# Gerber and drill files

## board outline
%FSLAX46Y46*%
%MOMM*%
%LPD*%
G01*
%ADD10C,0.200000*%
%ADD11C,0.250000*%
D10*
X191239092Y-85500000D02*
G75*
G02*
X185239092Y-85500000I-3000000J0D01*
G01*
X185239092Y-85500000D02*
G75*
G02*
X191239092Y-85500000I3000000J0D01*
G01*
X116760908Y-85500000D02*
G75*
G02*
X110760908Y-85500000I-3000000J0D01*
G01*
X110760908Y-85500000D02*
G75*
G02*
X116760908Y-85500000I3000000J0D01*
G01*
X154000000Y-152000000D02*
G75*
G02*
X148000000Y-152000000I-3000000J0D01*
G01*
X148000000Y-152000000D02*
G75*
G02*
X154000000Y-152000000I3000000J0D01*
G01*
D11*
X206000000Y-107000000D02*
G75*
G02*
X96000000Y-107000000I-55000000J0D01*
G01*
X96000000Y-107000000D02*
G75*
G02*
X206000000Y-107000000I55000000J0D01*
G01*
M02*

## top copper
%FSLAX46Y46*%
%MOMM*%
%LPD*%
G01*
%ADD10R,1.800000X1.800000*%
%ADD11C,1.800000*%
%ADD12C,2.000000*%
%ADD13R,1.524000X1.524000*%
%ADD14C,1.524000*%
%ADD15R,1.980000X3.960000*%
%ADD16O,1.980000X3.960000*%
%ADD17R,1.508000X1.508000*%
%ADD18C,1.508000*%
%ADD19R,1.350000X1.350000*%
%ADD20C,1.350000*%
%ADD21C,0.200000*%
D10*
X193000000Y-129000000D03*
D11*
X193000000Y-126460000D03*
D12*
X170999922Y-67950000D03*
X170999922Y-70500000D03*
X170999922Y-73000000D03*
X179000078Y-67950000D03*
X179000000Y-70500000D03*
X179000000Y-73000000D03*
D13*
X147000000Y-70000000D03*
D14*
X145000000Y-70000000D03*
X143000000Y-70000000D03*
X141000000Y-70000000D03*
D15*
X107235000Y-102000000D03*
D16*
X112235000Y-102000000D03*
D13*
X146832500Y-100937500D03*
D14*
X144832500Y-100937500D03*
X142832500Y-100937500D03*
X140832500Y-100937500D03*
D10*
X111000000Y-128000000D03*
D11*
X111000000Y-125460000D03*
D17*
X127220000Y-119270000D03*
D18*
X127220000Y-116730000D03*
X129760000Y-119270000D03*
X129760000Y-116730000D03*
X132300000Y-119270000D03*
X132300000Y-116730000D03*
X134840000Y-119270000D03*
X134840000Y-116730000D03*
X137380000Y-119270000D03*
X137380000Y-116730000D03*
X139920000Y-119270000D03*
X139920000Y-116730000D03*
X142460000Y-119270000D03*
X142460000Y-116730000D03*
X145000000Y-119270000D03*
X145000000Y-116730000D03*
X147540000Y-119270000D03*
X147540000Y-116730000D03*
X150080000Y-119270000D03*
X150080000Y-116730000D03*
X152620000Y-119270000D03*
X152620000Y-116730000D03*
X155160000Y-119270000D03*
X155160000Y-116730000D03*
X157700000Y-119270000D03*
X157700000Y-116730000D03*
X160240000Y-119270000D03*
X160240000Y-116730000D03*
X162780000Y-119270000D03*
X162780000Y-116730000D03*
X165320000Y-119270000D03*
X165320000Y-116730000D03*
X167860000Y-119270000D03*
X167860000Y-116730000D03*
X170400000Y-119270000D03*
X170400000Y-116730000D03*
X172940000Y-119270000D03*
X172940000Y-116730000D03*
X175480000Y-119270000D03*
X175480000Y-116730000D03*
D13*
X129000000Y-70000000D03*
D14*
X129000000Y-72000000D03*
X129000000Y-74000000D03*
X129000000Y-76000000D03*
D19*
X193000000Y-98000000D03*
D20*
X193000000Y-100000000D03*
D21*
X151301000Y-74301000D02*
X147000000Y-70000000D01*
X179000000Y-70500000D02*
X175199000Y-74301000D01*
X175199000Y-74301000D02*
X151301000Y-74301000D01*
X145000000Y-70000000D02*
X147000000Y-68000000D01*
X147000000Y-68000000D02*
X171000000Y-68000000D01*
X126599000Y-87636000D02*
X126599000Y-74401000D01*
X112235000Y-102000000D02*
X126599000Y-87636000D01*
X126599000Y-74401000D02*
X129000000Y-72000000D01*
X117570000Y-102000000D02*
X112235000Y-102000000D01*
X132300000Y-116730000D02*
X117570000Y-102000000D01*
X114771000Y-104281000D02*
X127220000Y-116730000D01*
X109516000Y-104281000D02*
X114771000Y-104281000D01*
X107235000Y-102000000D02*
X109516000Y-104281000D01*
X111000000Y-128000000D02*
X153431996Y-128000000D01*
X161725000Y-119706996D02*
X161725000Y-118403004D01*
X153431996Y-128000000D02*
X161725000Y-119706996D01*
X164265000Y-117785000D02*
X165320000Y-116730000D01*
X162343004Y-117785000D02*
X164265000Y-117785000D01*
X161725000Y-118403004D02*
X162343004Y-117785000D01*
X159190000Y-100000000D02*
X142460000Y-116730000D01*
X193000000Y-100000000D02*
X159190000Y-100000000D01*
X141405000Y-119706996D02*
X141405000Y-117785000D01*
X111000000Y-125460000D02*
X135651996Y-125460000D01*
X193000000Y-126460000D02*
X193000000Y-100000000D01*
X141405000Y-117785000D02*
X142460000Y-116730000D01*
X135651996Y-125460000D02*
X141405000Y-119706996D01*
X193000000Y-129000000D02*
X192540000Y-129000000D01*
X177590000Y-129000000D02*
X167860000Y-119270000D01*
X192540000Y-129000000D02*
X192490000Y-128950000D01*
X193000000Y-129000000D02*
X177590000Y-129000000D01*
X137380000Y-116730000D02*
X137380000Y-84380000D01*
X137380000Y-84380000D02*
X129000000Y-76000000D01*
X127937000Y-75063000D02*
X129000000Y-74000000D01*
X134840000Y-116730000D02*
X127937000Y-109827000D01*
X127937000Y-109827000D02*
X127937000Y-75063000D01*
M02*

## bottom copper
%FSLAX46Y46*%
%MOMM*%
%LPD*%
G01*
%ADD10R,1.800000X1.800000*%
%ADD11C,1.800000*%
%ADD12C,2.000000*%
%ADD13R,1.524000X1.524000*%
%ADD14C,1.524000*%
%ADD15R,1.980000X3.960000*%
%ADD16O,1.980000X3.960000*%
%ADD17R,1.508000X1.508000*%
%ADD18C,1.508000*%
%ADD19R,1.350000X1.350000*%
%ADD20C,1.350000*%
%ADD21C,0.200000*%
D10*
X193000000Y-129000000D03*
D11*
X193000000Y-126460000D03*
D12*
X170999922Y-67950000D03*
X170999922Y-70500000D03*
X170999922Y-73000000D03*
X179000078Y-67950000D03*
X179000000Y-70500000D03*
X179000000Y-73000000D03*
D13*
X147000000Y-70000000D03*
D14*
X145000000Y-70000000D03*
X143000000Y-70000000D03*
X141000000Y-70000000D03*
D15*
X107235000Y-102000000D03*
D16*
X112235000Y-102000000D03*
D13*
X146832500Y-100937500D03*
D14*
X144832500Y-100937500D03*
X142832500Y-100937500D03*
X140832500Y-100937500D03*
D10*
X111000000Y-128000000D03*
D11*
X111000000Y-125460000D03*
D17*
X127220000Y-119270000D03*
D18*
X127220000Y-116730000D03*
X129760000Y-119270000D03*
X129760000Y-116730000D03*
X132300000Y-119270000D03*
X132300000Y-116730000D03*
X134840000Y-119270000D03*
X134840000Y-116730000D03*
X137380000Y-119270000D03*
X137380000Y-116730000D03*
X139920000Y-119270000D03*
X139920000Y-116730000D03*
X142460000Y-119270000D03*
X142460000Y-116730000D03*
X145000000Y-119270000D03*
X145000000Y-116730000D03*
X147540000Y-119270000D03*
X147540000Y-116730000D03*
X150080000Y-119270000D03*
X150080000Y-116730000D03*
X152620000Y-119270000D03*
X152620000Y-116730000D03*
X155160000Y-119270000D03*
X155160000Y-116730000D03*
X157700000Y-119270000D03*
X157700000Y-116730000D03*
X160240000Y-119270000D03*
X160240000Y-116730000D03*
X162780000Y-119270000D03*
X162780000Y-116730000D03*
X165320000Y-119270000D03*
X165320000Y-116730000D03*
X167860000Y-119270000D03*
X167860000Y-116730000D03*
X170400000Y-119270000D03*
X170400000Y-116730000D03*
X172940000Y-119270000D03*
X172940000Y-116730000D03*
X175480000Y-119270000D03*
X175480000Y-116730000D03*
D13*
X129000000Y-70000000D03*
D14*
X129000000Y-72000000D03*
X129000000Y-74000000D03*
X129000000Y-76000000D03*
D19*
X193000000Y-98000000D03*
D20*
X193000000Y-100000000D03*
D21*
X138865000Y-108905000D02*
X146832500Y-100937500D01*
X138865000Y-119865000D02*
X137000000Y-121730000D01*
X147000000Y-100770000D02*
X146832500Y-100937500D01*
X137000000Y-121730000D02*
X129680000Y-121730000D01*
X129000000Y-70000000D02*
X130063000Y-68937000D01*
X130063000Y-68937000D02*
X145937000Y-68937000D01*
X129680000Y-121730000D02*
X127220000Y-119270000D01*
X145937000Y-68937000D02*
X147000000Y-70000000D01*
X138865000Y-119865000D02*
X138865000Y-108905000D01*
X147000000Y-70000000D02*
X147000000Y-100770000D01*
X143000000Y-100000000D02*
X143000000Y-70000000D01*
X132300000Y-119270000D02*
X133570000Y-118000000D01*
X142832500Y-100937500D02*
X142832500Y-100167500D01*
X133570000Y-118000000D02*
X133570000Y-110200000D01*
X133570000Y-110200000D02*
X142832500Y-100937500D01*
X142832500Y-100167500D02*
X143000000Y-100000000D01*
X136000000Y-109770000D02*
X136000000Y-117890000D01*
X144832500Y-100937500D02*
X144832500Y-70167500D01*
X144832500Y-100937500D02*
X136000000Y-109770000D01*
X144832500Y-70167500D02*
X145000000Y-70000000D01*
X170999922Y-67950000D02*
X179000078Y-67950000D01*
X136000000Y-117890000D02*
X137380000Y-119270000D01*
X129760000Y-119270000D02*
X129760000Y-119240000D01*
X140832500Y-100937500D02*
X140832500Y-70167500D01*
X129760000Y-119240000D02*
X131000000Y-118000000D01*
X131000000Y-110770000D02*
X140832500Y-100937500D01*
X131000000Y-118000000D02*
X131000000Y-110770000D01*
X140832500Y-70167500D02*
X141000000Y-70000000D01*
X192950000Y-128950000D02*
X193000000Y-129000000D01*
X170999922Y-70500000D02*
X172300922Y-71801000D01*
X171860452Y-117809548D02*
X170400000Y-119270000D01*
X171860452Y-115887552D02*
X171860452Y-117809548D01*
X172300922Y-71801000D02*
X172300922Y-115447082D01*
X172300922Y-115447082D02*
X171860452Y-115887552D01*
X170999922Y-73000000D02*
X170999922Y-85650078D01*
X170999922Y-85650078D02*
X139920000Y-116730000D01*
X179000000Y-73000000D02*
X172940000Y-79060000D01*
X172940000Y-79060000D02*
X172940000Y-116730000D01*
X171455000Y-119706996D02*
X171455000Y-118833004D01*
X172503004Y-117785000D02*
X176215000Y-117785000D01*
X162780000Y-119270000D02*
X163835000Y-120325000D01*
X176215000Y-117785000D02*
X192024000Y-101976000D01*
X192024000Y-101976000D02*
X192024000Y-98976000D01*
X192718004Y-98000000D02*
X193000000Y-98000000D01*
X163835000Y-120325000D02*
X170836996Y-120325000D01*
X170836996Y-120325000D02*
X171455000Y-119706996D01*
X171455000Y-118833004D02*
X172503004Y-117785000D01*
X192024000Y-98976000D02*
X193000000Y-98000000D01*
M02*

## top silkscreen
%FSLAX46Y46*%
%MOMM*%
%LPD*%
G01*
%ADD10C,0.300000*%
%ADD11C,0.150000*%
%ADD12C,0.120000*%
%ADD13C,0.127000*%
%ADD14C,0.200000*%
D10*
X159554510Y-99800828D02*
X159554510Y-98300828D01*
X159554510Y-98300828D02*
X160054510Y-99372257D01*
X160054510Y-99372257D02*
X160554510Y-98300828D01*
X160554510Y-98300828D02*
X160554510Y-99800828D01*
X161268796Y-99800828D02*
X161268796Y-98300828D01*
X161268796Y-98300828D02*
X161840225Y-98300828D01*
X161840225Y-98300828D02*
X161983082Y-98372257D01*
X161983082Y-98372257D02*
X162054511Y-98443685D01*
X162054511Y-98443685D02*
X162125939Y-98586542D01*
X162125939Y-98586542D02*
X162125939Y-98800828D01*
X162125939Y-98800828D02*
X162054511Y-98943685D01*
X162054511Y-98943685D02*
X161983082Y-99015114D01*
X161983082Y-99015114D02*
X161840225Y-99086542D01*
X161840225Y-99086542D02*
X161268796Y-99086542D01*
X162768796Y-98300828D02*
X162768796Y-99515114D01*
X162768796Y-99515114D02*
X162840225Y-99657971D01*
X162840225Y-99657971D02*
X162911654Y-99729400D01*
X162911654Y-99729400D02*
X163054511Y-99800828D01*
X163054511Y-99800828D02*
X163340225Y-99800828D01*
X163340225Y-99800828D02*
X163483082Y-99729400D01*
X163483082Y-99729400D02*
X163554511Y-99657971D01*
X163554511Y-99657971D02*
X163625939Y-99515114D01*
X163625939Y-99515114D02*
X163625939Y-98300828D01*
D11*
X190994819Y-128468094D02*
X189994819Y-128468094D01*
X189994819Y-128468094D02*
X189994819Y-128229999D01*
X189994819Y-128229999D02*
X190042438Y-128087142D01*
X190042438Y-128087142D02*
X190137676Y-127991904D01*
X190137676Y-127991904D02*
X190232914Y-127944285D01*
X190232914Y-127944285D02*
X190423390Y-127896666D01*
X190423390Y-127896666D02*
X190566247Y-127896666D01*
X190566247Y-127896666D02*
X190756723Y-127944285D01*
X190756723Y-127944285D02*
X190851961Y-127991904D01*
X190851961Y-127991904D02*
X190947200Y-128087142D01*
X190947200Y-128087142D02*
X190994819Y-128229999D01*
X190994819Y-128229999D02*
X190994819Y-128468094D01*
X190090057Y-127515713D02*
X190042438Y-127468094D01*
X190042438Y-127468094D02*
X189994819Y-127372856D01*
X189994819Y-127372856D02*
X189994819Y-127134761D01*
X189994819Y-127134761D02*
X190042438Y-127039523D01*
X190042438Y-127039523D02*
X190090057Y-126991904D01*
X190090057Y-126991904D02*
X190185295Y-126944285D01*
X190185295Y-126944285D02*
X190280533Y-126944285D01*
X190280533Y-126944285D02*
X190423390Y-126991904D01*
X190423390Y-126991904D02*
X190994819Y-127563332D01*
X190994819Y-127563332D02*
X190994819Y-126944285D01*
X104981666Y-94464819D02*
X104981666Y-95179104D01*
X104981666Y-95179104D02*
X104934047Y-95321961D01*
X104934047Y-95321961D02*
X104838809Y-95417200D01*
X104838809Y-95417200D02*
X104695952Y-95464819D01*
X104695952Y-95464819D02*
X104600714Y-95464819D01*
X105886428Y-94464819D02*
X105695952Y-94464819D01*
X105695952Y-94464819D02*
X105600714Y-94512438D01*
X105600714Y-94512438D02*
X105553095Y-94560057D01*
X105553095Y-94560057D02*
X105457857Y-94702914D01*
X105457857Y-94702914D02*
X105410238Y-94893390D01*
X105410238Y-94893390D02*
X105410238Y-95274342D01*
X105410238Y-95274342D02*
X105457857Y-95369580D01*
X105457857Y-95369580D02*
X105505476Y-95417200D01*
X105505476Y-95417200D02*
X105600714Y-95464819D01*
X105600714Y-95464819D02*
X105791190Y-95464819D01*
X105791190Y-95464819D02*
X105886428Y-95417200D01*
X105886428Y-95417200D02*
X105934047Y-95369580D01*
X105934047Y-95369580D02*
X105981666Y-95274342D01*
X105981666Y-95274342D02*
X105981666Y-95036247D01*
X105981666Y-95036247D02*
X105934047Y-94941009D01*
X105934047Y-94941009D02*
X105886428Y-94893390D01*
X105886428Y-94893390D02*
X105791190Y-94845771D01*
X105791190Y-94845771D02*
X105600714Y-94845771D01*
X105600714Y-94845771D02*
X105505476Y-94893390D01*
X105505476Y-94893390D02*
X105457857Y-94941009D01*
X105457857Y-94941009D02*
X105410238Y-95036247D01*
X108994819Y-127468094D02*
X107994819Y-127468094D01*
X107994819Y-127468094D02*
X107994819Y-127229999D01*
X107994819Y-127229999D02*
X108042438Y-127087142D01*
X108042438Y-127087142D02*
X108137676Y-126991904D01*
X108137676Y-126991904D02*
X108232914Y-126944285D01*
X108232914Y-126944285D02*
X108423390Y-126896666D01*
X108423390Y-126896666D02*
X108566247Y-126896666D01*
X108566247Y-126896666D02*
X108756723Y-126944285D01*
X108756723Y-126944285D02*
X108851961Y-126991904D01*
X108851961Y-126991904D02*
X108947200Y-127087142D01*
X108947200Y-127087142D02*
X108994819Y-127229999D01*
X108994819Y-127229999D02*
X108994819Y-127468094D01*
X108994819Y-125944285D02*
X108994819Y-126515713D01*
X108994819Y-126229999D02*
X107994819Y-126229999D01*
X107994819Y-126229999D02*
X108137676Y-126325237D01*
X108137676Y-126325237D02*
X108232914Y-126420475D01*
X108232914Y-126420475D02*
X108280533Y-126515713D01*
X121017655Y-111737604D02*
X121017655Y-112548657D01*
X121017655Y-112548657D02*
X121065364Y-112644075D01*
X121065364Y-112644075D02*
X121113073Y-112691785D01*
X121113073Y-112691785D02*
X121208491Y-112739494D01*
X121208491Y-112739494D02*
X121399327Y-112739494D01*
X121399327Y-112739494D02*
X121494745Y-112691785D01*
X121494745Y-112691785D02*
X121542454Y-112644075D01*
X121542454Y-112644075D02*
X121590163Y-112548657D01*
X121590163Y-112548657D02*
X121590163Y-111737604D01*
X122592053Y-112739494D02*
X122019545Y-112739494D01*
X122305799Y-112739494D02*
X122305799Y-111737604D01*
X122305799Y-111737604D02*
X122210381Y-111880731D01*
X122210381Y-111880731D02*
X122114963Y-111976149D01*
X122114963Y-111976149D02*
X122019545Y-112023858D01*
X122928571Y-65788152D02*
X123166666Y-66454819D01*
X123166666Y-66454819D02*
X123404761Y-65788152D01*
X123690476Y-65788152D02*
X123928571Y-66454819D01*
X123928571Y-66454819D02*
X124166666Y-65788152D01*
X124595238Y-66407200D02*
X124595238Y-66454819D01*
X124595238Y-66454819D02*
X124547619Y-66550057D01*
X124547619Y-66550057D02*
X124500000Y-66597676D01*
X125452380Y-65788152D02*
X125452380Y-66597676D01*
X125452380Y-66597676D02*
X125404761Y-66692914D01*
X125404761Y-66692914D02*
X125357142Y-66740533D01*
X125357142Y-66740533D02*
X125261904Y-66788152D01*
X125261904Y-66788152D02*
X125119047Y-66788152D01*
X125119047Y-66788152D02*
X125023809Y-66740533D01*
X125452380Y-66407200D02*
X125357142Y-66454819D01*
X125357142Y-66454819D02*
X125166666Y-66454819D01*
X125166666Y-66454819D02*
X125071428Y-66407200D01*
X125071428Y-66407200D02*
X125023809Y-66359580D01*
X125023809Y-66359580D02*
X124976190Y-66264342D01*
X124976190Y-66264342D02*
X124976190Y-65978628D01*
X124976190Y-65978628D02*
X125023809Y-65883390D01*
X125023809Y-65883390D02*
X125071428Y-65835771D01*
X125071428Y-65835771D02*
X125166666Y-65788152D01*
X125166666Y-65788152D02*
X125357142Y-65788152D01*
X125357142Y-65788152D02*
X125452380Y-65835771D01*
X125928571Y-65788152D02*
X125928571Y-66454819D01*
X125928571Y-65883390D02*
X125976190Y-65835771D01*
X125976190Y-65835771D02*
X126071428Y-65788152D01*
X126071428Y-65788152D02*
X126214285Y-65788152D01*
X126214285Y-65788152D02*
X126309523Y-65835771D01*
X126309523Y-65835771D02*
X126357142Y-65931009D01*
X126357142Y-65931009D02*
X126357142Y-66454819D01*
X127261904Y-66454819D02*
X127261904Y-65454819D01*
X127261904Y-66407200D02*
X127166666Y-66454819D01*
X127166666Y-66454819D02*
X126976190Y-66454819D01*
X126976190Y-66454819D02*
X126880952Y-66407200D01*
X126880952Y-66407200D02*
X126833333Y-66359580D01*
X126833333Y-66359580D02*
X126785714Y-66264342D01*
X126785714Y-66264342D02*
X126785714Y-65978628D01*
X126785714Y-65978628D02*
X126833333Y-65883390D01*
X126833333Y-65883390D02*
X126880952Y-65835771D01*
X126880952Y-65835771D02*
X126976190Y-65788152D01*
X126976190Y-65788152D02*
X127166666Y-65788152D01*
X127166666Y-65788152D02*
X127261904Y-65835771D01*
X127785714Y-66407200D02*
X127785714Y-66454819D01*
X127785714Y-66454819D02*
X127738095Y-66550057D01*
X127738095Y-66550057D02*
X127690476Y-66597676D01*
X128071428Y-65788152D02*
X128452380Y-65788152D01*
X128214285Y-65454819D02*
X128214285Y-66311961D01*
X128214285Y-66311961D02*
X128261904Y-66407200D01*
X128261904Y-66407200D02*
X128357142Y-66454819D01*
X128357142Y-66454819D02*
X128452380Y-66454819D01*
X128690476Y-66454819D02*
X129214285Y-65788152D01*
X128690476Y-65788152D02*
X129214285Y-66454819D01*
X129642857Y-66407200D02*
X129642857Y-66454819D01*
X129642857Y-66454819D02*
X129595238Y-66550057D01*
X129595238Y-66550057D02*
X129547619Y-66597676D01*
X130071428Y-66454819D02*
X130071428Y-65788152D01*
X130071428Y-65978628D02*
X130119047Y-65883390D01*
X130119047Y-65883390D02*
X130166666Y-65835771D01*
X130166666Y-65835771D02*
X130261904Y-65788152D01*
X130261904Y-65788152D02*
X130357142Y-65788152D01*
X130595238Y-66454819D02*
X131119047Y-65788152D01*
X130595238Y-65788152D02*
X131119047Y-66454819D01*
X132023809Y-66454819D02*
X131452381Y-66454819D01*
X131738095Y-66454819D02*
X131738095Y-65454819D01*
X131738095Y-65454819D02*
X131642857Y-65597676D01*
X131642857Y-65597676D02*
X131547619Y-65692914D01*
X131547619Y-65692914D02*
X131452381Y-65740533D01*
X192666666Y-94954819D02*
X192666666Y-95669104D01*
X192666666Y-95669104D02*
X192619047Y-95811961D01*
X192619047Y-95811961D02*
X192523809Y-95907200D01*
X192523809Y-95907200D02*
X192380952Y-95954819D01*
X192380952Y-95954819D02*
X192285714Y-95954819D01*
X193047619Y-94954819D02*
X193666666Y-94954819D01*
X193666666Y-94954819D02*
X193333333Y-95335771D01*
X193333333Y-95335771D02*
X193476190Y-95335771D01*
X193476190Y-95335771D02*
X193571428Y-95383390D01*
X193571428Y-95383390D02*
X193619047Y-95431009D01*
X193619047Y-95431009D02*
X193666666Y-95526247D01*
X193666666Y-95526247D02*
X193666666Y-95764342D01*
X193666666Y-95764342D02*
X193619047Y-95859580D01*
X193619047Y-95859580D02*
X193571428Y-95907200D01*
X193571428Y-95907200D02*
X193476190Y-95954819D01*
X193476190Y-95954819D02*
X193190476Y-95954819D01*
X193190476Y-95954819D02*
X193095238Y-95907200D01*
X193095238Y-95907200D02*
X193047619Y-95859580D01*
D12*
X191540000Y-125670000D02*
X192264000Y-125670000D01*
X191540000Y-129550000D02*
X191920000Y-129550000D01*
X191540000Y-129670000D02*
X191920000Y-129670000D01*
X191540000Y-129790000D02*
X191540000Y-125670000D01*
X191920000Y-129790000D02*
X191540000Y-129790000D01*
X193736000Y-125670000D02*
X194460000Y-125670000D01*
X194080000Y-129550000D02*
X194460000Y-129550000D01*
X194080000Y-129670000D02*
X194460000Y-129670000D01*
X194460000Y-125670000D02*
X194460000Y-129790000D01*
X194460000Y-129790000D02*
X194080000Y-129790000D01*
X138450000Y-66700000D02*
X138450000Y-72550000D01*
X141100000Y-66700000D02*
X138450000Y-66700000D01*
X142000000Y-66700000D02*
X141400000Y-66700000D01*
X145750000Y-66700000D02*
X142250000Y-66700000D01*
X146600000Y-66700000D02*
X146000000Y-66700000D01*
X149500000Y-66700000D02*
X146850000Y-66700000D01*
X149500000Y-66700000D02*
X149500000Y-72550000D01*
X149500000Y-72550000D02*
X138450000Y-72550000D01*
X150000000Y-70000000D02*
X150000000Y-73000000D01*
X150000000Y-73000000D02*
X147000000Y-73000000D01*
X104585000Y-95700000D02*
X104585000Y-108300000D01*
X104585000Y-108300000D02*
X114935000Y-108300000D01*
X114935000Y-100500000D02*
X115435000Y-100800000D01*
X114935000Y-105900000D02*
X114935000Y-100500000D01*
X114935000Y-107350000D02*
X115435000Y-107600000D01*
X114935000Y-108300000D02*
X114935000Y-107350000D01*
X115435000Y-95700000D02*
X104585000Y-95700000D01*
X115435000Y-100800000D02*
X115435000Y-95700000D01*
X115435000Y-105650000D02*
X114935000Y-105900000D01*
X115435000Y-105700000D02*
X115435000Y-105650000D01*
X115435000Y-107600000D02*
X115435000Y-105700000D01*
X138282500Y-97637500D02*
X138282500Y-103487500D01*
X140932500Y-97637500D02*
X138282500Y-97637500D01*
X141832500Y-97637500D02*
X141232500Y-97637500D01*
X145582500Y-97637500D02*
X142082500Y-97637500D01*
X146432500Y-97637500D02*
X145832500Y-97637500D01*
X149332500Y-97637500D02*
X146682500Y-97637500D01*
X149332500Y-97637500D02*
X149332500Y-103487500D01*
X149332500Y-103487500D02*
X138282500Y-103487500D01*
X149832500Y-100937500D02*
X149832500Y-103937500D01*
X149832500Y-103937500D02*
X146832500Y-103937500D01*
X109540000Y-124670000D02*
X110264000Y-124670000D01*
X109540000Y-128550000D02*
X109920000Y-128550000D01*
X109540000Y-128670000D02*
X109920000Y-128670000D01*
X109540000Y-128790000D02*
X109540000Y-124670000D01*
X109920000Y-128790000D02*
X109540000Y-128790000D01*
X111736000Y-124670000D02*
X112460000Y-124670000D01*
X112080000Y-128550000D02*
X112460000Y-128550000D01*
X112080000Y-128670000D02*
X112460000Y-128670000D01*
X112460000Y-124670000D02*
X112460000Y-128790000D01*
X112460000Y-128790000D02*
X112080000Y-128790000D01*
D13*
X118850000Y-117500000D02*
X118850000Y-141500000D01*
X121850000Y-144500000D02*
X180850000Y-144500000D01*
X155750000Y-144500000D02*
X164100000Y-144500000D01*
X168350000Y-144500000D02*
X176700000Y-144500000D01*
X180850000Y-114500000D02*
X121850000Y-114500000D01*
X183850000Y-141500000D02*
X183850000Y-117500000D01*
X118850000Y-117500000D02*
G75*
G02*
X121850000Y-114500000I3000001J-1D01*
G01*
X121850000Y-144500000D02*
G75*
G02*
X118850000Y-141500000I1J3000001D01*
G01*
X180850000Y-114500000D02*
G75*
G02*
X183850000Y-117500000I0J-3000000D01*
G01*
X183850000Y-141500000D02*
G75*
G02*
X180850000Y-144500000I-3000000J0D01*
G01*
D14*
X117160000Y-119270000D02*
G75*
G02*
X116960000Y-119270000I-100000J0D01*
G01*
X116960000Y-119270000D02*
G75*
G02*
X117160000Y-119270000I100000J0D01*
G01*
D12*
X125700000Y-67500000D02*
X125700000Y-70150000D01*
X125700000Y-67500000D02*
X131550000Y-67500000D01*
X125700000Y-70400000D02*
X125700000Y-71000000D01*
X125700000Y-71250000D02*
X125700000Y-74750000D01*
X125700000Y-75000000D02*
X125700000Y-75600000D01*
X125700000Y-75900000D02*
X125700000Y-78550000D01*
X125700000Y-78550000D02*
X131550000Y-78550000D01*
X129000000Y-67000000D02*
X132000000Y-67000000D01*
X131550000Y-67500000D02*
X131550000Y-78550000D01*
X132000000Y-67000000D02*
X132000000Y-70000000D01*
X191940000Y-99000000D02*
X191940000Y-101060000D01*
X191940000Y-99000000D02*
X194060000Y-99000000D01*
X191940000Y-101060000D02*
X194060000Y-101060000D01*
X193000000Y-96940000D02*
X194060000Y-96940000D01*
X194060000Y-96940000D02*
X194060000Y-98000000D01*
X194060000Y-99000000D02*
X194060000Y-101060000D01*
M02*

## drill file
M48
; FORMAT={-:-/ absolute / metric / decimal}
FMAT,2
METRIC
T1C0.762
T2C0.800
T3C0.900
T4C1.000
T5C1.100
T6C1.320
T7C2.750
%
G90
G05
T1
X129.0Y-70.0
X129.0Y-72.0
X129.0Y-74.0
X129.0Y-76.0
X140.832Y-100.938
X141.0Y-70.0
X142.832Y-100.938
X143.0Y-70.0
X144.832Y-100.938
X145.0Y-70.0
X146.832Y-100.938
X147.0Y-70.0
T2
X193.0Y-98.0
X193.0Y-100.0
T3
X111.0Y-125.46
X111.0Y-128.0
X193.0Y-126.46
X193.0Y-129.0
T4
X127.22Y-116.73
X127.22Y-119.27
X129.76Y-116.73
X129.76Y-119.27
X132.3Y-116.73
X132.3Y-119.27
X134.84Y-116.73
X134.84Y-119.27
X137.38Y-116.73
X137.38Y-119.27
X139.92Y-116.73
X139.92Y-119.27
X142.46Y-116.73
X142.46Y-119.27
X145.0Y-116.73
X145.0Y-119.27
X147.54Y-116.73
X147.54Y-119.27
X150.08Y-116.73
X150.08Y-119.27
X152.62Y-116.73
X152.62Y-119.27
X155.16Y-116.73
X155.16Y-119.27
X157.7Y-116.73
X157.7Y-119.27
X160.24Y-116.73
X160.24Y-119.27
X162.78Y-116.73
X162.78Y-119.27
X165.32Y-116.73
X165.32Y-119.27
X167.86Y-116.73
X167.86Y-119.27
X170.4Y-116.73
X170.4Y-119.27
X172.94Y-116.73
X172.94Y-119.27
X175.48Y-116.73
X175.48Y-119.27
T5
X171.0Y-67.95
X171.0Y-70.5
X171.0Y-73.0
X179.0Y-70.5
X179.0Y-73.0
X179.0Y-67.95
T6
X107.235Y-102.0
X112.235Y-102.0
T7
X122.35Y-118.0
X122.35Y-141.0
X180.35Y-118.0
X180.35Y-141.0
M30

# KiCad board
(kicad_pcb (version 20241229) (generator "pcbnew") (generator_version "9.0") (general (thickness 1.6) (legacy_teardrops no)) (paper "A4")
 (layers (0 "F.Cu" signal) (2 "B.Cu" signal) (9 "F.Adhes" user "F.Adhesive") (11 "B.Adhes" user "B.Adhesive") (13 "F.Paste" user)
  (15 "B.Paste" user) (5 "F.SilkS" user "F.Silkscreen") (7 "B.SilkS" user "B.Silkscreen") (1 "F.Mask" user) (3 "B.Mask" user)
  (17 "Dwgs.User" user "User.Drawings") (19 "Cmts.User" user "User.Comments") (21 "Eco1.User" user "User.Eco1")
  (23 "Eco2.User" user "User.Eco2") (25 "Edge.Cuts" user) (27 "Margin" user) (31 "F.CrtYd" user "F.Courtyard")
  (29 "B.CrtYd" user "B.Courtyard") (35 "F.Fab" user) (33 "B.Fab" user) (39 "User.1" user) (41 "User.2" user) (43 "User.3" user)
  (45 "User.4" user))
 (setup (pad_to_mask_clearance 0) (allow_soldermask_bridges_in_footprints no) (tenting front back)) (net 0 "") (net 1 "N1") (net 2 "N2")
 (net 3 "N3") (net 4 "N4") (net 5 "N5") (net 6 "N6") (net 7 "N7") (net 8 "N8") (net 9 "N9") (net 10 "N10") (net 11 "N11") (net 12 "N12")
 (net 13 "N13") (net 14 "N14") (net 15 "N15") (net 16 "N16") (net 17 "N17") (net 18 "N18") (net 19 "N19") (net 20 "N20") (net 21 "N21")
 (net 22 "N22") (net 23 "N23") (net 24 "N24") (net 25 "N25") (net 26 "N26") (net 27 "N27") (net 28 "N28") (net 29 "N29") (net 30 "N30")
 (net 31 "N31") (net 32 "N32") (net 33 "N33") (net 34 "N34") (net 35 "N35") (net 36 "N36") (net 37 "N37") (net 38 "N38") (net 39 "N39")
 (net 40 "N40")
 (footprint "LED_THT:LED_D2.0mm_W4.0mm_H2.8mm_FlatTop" (layer "F.Cu") (at 193 129 90)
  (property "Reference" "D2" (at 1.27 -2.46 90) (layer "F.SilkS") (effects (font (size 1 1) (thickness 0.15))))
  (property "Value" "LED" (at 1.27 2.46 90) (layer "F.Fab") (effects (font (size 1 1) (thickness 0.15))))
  (fp_line (start 3.33 -1.46) (end 3.33 -0.736) (stroke (width 0.12) (type solid)) (layer "F.SilkS"))
  (fp_line (start -0.55 -1.46) (end -0.55 -1.08) (stroke (width 0.12) (type solid)) (layer "F.SilkS"))
  (fp_line (start -0.67 -1.46) (end -0.67 -1.08) (stroke (width 0.12) (type solid)) (layer "F.SilkS"))
  (fp_line (start -0.79 -1.46) (end 3.33 -1.46) (stroke (width 0.12) (type solid)) (layer "F.SilkS"))
  (fp_line (start -0.79 -1.08) (end -0.79 -1.46) (stroke (width 0.12) (type solid)) (layer "F.SilkS"))
  (fp_line (start 3.33 0.736) (end 3.33 1.46) (stroke (width 0.12) (type solid)) (layer "F.SilkS"))
  (fp_line (start -0.55 1.08) (end -0.55 1.46) (stroke (width 0.12) (type solid)) (layer "F.SilkS"))
  (fp_line (start -0.67 1.08) (end -0.67 1.46) (stroke (width 0.12) (type solid)) (layer "F.SilkS"))
  (fp_line (start 3.33 1.46) (end -0.79 1.46) (stroke (width 0.12) (type solid)) (layer "F.SilkS"))
  (fp_line (start -0.79 1.46) (end -0.79 1.08) (stroke (width 0.12) (type solid)) (layer "F.SilkS"))
  (pad "1" thru_hole rect (at 0 0 90) (size 1.8 1.8) (drill 0.9) (layers "*.Cu" "*.Mask") (remove_unused_layers no) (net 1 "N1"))
  (pad "2" thru_hole circle (at 2.54 0 90) (size 1.8 1.8) (drill 0.9) (layers "*.Cu" "*.Mask") (remove_unused_layers no) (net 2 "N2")))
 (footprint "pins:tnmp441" (layer "F.Cu") (at 174.999922 70.5)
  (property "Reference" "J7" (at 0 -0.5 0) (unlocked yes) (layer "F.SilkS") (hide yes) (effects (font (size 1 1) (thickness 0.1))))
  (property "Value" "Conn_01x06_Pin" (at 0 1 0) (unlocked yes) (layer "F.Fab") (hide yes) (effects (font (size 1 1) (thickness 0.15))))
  (pad "1" thru_hole circle (at -4 -2.55) (size 2 2) (drill 1.1) (layers "*.Cu" "*.Mask") (remove_unused_layers no) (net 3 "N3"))
  (pad "2" thru_hole circle (at -4 0) (size 2 2) (drill 1.1) (layers "*.Cu" "*.Mask") (remove_unused_layers no) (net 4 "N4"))
  (pad "3" thru_hole circle (at -4 2.5) (size 2 2) (drill 1.1) (layers "*.Cu" "*.Mask") (remove_unused_layers no) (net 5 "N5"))
  (pad "4" thru_hole circle (at 4.000156 -2.55) (size 2 2) (drill 1.1) (layers "*.Cu" "*.Mask") (remove_unused_layers no) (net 3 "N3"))
  (pad "5" thru_hole circle (at 4.000078 0) (size 2 2) (drill 1.1) (layers "*.Cu" "*.Mask") (remove_unused_layers no) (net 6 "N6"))
  (pad "6" thru_hole circle (at 4.000078 2.5) (size 2 2) (drill 1.1) (layers "*.Cu" "*.Mask") (remove_unused_layers no) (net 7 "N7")))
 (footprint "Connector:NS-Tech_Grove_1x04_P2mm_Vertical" (layer "F.Cu") (at 147 70 -90)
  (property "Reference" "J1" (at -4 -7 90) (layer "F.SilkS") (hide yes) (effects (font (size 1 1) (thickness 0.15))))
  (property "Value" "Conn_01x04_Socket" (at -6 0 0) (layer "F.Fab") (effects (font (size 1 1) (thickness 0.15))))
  (fp_line (start -3.3 8.55) (end 2.55 8.55) (stroke (width 0.12) (type solid)) (layer "F.SilkS"))
  (fp_line (start -3.3 5.9) (end -3.3 8.55) (stroke (width 0.12) (type solid)) (layer "F.SilkS"))
  (fp_line (start -3.3 5) (end -3.3 5.6) (stroke (width 0.12) (type solid)) (layer "F.SilkS"))
  (fp_line (start -3.3 1.25) (end -3.3 4.75) (stroke (width 0.12) (type solid)) (layer "F.SilkS"))
  (fp_line (start -3.3 0.4) (end -3.3 1) (stroke (width 0.12) (type solid)) (layer "F.SilkS"))
  (fp_line (start -3.3 -2.5) (end -3.3 0.15) (stroke (width 0.12) (type solid)) (layer "F.SilkS"))
  (fp_line (start -3.3 -2.5) (end 2.55 -2.5) (stroke (width 0.12) (type solid)) (layer "F.SilkS"))
  (fp_line (start 2.55 -2.5) (end 2.55 8.55) (stroke (width 0.12) (type solid)) (layer "F.SilkS"))
  (fp_line (start 0 -3) (end 3 -3) (stroke (width 0.12) (type solid)) (layer "F.SilkS"))
  (fp_line (start 3 -3) (end 3 0) (stroke (width 0.12) (type solid)) (layer "F.SilkS"))
  (pad "1" thru_hole rect (at 0 0 270) (size 1.524 1.524) (drill 0.762) (layers "*.Cu" "*.Mask") (remove_unused_layers no) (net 6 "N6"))
  (pad "2" thru_hole circle (at 0 2 270) (size 1.524 1.524) (drill 0.762) (layers "*.Cu" "*.Mask") (remove_unused_layers no) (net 3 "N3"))
  (pad "3" thru_hole circle (at 0 4 270) (size 1.524 1.524) (drill 0.762) (layers "*.Cu" "*.Mask") (remove_unused_layers no) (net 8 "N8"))
  (pad "4" thru_hole circle (at 0 6 270) (size 1.524 1.524) (drill 0.762) (layers "*.Cu" "*.Mask") (remove_unused_layers no) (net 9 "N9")))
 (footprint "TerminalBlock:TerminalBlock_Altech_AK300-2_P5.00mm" (layer "F.Cu") (at 107.235 102)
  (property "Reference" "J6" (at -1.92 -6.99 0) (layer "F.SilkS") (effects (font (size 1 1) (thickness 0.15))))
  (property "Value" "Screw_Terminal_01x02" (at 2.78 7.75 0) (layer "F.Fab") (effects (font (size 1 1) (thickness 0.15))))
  (fp_line (start -2.65 -6.3) (end -2.65 6.3) (stroke (width 0.12) (type solid)) (layer "F.SilkS"))
  (fp_line (start -2.65 6.3) (end 7.7 6.3) (stroke (width 0.12) (type solid)) (layer "F.SilkS"))
  (fp_line (start 7.7 -1.5) (end 8.2 -1.2) (stroke (width 0.12) (type solid)) (layer "F.SilkS"))
  (fp_line (start 7.7 3.9) (end 7.7 -1.5) (stroke (width 0.12) (type solid)) (layer "F.SilkS"))
  (fp_line (start 7.7 5.35) (end 8.2 5.6) (stroke (width 0.12) (type solid)) (layer "F.SilkS"))
  (fp_line (start 7.7 6.3) (end 7.7 5.35) (stroke (width 0.12) (type solid)) (layer "F.SilkS"))
  (fp_line (start 8.2 -6.3) (end -2.65 -6.3) (stroke (width 0.12) (type solid)) (layer "F.SilkS"))
  (fp_line (start 8.2 -1.2) (end 8.2 -6.3) (stroke (width 0.12) (type solid)) (layer "F.SilkS"))
  (fp_line (start 8.2 3.65) (end 7.7 3.9) (stroke (width 0.12) (type solid)) (layer "F.SilkS"))
  (fp_line (start 8.2 3.7) (end 8.2 3.65) (stroke (width 0.12) (type solid)) (layer "F.SilkS"))
  (fp_line (start 8.2 5.6) (end 8.2 3.7) (stroke (width 0.12) (type solid)) (layer "F.SilkS"))
  (pad "1" thru_hole rect (at 0 0) (size 1.98 3.96) (drill 1.32) (layers "*.Cu" "*.Mask") (remove_unused_layers no) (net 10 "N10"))
  (pad "2" thru_hole oval (at 5 0) (size 1.98 3.96) (drill 1.32) (layers "*.Cu" "*.Mask") (remove_unused_layers no) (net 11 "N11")))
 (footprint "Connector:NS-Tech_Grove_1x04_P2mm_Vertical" (layer "F.Cu") (at 146.8325 100.9375 -90)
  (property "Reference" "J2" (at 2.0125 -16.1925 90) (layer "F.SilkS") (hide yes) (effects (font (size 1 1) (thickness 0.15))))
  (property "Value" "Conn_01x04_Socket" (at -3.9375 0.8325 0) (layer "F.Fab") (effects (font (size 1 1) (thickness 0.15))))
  (fp_line (start -3.3 8.55) (end 2.55 8.55) (stroke (width 0.12) (type solid)) (layer "F.SilkS"))
  (fp_line (start -3.3 5.9) (end -3.3 8.55) (stroke (width 0.12) (type solid)) (layer "F.SilkS"))
  (fp_line (start -3.3 5) (end -3.3 5.6) (stroke (width 0.12) (type solid)) (layer "F.SilkS"))
  (fp_line (start -3.3 1.25) (end -3.3 4.75) (stroke (width 0.12) (type solid)) (layer "F.SilkS"))
  (fp_line (start -3.3 0.4) (end -3.3 1) (stroke (width 0.12) (type solid)) (layer "F.SilkS"))
  (fp_line (start -3.3 -2.5) (end -3.3 0.15) (stroke (width 0.12) (type solid)) (layer "F.SilkS"))
  (fp_line (start -3.3 -2.5) (end 2.55 -2.5) (stroke (width 0.12) (type solid)) (layer "F.SilkS"))
  (fp_line (start 2.55 -2.5) (end 2.55 8.55) (stroke (width 0.12) (type solid)) (layer "F.SilkS"))
  (fp_line (start 0 -3) (end 3 -3) (stroke (width 0.12) (type solid)) (layer "F.SilkS"))
  (fp_line (start 3 -3) (end 3 0) (stroke (width 0.12) (type solid)) (layer "F.SilkS"))
  (pad "1" thru_hole rect (at 0 0 270) (size 1.524 1.524) (drill 0.762) (layers "*.Cu" "*.Mask") (remove_unused_layers no) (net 6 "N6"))
  (pad "2" thru_hole circle (at 0 2 270) (size 1.524 1.524) (drill 0.762) (layers "*.Cu" "*.Mask") (remove_unused_layers no) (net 3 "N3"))
  (pad "3" thru_hole circle (at 0 4 270) (size 1.524 1.524) (drill 0.762) (layers "*.Cu" "*.Mask") (remove_unused_layers no) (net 8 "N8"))
  (pad "4" thru_hole circle (at 0 6 270) (size 1.524 1.524) (drill 0.762) (layers "*.Cu" "*.Mask") (remove_unused_layers no) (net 9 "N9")))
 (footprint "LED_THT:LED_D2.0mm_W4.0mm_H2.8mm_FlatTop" (layer "F.Cu") (at 111 128 90)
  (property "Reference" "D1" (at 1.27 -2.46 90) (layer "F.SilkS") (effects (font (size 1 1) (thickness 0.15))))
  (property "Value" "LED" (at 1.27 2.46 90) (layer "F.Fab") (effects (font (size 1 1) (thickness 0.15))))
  (fp_line (start 3.33 -1.46) (end 3.33 -0.736) (stroke (width 0.12) (type solid)) (layer "F.SilkS"))
  (fp_line (start -0.55 -1.46) (end -0.55 -1.08) (stroke (width 0.12) (type solid)) (layer "F.SilkS"))
  (fp_line (start -0.67 -1.46) (end -0.67 -1.08) (stroke (width 0.12) (type solid)) (layer "F.SilkS"))
  (fp_line (start -0.79 -1.46) (end 3.33 -1.46) (stroke (width 0.12) (type solid)) (layer "F.SilkS"))
  (fp_line (start -0.79 -1.08) (end -0.79 -1.46) (stroke (width 0.12) (type solid)) (layer "F.SilkS"))
  (fp_line (start 3.33 0.736) (end 3.33 1.46) (stroke (width 0.12) (type solid)) (layer "F.SilkS"))
  (fp_line (start -0.55 1.08) (end -0.55 1.46) (stroke (width 0.12) (type solid)) (layer "F.SilkS"))
  (fp_line (start -0.67 1.08) (end -0.67 1.46) (stroke (width 0.12) (type solid)) (layer "F.SilkS"))
  (fp_line (start 3.33 1.46) (end -0.79 1.46) (stroke (width 0.12) (type solid)) (layer "F.SilkS"))
  (fp_line (start -0.79 1.46) (end -0.79 1.08) (stroke (width 0.12) (type solid)) (layer "F.SilkS"))
  (pad "1" thru_hole rect (at 0 0 90) (size 1.8 1.8) (drill 0.9) (layers "*.Cu" "*.Mask") (remove_unused_layers no) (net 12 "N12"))
  (pad "2" thru_hole circle (at 2.54 0 90) (size 1.8 1.8) (drill 0.9) (layers "*.Cu" "*.Mask") (remove_unused_layers no) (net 2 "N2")))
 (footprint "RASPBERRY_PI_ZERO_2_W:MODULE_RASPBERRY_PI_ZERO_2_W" (layer "F.Cu") (at 151.35 129.5)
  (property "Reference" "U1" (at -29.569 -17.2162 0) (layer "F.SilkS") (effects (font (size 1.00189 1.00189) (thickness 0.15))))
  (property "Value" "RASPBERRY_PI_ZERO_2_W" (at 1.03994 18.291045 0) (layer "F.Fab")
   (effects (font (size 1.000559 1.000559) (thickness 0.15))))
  (fp_line (start -32.5 -12) (end -32.5 12) (stroke (width 0.127) (type solid)) (layer "F.SilkS"))
  (fp_line (start -29.5 15) (end 29.5 15) (stroke (width 0.127) (type solid)) (layer "F.SilkS"))
  (fp_line (start 4.4 15) (end 12.75 15) (stroke (width 0.127) (type solid)) (layer "F.SilkS"))
  (fp_line (start 17 15) (end 25.35 15) (stroke (width 0.127) (type solid)) (layer "F.SilkS"))
  (fp_line (start 29.5 -15) (end -29.5 -15) (stroke (width 0.127) (type solid)) (layer "F.SilkS"))
  (fp_line (start 32.5 12) (end 32.5 -12) (stroke (width 0.127) (type solid)) (layer "F.SilkS"))
  (fp_arc (start -32.5 -12) (mid -31.62132 -14.12132) (end -29.5 -15) (stroke (width 0.127) (type solid)) (layer "F.SilkS"))
  (fp_arc (start -29.5 15) (mid -31.62132 14.12132) (end -32.5 12) (stroke (width 0.127) (type solid)) (layer "F.SilkS"))
  (fp_arc (start 29.5 -15) (mid 31.62132 -14.12132) (end 32.5 -12) (stroke (width 0.127) (type solid)) (layer "F.SilkS"))
  (fp_arc (start 32.5 12) (mid 31.62132 14.12132) (end 29.5 15) (stroke (width 0.127) (type solid)) (layer "F.SilkS"))
  (fp_circle (center -34.29 -10.23) (end -34.19 -10.23) (stroke (width 0.2) (type solid)) (fill no) (layer "F.SilkS"))
  (pad "" np_thru_hole circle (at -29 -11.5) (size 2.75 2.75) (drill 2.75) (layers "*.Cu" "*.Mask"))
  (pad "" np_thru_hole circle (at -29 11.5) (size 2.75 2.75) (drill 2.75) (layers "*.Cu" "*.Mask"))
  (pad "" np_thru_hole circle (at 29 -11.5) (size 2.75 2.75) (drill 2.75) (layers "*.Cu" "*.Mask"))
  (pad "" np_thru_hole circle (at 29 11.5) (size 2.75 2.75) (drill 2.75) (layers "*.Cu" "*.Mask"))
  (pad "1" thru_hole rect (at -24.13 -10.23) (size 1.508 1.508) (drill 1) (layers "*.Cu" "*.Mask") (remove_unused_layers no) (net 6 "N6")
   (solder_mask_margin 0.102))
  (pad "2" thru_hole circle (at -24.13 -12.77) (size 1.508 1.508) (drill 1) (layers "*.Cu" "*.Mask") (remove_unused_layers no)
   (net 10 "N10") (solder_mask_margin 0.102))
  (pad "3" thru_hole circle (at -21.59 -10.23) (size 1.508 1.508) (drill 1) (layers "*.Cu" "*.Mask") (remove_unused_layers no) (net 9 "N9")
   (solder_mask_margin 0.102))
  (pad "4" thru_hole circle (at -21.59 -12.77) (size 1.508 1.508) (drill 1) (layers "*.Cu" "*.Mask") (remove_unused_layers no)
   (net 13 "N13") (solder_mask_margin 0.102))
  (pad "5" thru_hole circle (at -19.05 -10.23) (size 1.508 1.508) (drill 1) (layers "*.Cu" "*.Mask") (remove_unused_layers no) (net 8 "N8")
   (solder_mask_margin 0.102))
  (pad "6" thru_hole circle (at -19.05 -12.77) (size 1.508 1.508) (drill 1) (layers "*.Cu" "*.Mask") (remove_unused_layers no)
   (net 11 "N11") (solder_mask_margin 0.102))
  (pad "7" thru_hole circle (at -16.51 -10.23) (size 1.508 1.508) (drill 1) (layers "*.Cu" "*.Mask") (remove_unused_layers no)
   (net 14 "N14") (solder_mask_margin 0.102))
  (pad "8" thru_hole circle (at -16.51 -12.77) (size 1.508 1.508) (drill 1) (layers "*.Cu" "*.Mask") (remove_unused_layers no)
   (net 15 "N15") (solder_mask_margin 0.102))
  (pad "9" thru_hole circle (at -13.97 -10.23) (size 1.508 1.508) (drill 1) (layers "*.Cu" "*.Mask") (remove_unused_layers no) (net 3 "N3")
   (solder_mask_margin 0.102))
  (pad "10" thru_hole circle (at -13.97 -12.77) (size 1.508 1.508) (drill 1) (layers "*.Cu" "*.Mask") (remove_unused_layers no)
   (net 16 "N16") (solder_mask_margin 0.102))
  (pad "11" thru_hole circle (at -11.43 -10.23) (size 1.508 1.508) (drill 1) (layers "*.Cu" "*.Mask") (remove_unused_layers no)
   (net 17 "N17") (solder_mask_margin 0.102))
  (pad "12" thru_hole circle (at -11.43 -12.77) (size 1.508 1.508) (drill 1) (layers "*.Cu" "*.Mask") (remove_unused_layers no) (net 5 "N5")
   (solder_mask_margin 0.102))
  (pad "13" thru_hole circle (at -8.89 -10.23) (size 1.508 1.508) (drill 1) (layers "*.Cu" "*.Mask") (remove_unused_layers no)
   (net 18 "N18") (solder_mask_margin 0.102))
  (pad "14" thru_hole circle (at -8.89 -12.77) (size 1.508 1.508) (drill 1) (layers "*.Cu" "*.Mask") (remove_unused_layers no) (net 2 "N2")
   (solder_mask_margin 0.102))
  (pad "15" thru_hole circle (at -6.35 -10.23) (size 1.508 1.508) (drill 1) (layers "*.Cu" "*.Mask") (remove_unused_layers no)
   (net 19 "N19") (solder_mask_margin 0.102))
  (pad "16" thru_hole circle (at -6.35 -12.77) (size 1.508 1.508) (drill 1) (layers "*.Cu" "*.Mask") (remove_unused_layers no)
   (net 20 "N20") (solder_mask_margin 0.102))
  (pad "17" thru_hole circle (at -3.81 -10.23) (size 1.508 1.508) (drill 1) (layers "*.Cu" "*.Mask") (remove_unused_layers no)
   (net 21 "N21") (solder_mask_margin 0.102))
  (pad "18" thru_hole circle (at -3.81 -12.77) (size 1.508 1.508) (drill 1) (layers "*.Cu" "*.Mask") (remove_unused_layers no)
   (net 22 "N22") (solder_mask_margin 0.102))
  (pad "19" thru_hole circle (at -1.27 -10.23) (size 1.508 1.508) (drill 1) (layers "*.Cu" "*.Mask") (remove_unused_layers no)
   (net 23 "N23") (solder_mask_margin 0.102))
  (pad "20" thru_hole circle (at -1.27 -12.77) (size 1.508 1.508) (drill 1) (layers "*.Cu" "*.Mask") (remove_unused_layers no)
   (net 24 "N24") (solder_mask_margin 0.102))
  (pad "21" thru_hole circle (at 1.27 -10.23) (size 1.508 1.508) (drill 1) (layers "*.Cu" "*.Mask") (remove_unused_layers no) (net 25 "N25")
   (solder_mask_margin 0.102))
  (pad "22" thru_hole circle (at 1.27 -12.77) (size 1.508 1.508) (drill 1) (layers "*.Cu" "*.Mask") (remove_unused_layers no) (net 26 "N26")
   (solder_mask_margin 0.102))
  (pad "23" thru_hole circle (at 3.81 -10.23) (size 1.508 1.508) (drill 1) (layers "*.Cu" "*.Mask") (remove_unused_layers no) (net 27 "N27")
   (solder_mask_margin 0.102))
  (pad "24" thru_hole circle (at 3.81 -12.77) (size 1.508 1.508) (drill 1) (layers "*.Cu" "*.Mask") (remove_unused_layers no) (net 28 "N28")
   (solder_mask_margin 0.102))
  (pad "25" thru_hole circle (at 6.35 -10.23) (size 1.508 1.508) (drill 1) (layers "*.Cu" "*.Mask") (remove_unused_layers no) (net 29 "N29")
   (solder_mask_margin 0.102))
  (pad "26" thru_hole circle (at 6.35 -12.77) (size 1.508 1.508) (drill 1) (layers "*.Cu" "*.Mask") (remove_unused_layers no) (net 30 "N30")
   (solder_mask_margin 0.102))
  (pad "27" thru_hole circle (at 8.89 -10.23) (size 1.508 1.508) (drill 1) (layers "*.Cu" "*.Mask") (remove_unused_layers no) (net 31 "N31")
   (solder_mask_margin 0.102))
  (pad "28" thru_hole circle (at 8.89 -12.77) (size 1.508 1.508) (drill 1) (layers "*.Cu" "*.Mask") (remove_unused_layers no) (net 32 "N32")
   (solder_mask_margin 0.102))
  (pad "29" thru_hole circle (at 11.43 -10.23) (size 1.508 1.508) (drill 1) (layers "*.Cu" "*.Mask") (remove_unused_layers no)
   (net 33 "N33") (solder_mask_margin 0.102))
  (pad "30" thru_hole circle (at 11.43 -12.77) (size 1.508 1.508) (drill 1) (layers "*.Cu" "*.Mask") (remove_unused_layers no)
   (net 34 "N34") (solder_mask_margin 0.102))
  (pad "31" thru_hole circle (at 13.97 -10.23) (size 1.508 1.508) (drill 1) (layers "*.Cu" "*.Mask") (remove_unused_layers no)
   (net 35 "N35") (solder_mask_margin 0.102))
  (pad "32" thru_hole circle (at 13.97 -12.77) (size 1.508 1.508) (drill 1) (layers "*.Cu" "*.Mask") (remove_unused_layers no)
   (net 12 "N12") (solder_mask_margin 0.102))
  (pad "33" thru_hole circle (at 16.51 -10.23) (size 1.508 1.508) (drill 1) (layers "*.Cu" "*.Mask") (remove_unused_layers no) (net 1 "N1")
   (solder_mask_margin 0.102))
  (pad "34" thru_hole circle (at 16.51 -12.77) (size 1.508 1.508) (drill 1) (layers "*.Cu" "*.Mask") (remove_unused_layers no)
   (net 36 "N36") (solder_mask_margin 0.102))
  (pad "35" thru_hole circle (at 19.05 -10.23) (size 1.508 1.508) (drill 1) (layers "*.Cu" "*.Mask") (remove_unused_layers no) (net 4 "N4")
   (solder_mask_margin 0.102))
  (pad "36" thru_hole circle (at 19.05 -12.77) (size 1.508 1.508) (drill 1) (layers "*.Cu" "*.Mask") (remove_unused_layers no)
   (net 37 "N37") (solder_mask_margin 0.102))
  (pad "37" thru_hole circle (at 21.59 -10.23) (size 1.508 1.508) (drill 1) (layers "*.Cu" "*.Mask") (remove_unused_layers no)
   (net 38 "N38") (solder_mask_margin 0.102))
  (pad "38" thru_hole circle (at 21.59 -12.77) (size 1.508 1.508) (drill 1) (layers "*.Cu" "*.Mask") (remove_unused_layers no) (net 7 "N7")
   (solder_mask_margin 0.102))
  (pad "39" thru_hole circle (at 24.13 -10.23) (size 1.508 1.508) (drill 1) (layers "*.Cu" "*.Mask") (remove_unused_layers no)
   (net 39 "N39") (solder_mask_margin 0.102))
  (pad "40" thru_hole circle (at 24.13 -12.77) (size 1.508 1.508) (drill 1) (layers "*.Cu" "*.Mask") (remove_unused_layers no)
   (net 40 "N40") (solder_mask_margin 0.102)))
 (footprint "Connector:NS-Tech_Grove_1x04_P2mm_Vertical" (layer "F.Cu") (at 129 70)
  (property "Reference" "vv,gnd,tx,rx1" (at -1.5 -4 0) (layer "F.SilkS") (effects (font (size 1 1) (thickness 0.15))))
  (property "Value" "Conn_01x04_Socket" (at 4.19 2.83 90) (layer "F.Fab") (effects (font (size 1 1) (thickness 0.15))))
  (fp_line (start -3.3 -2.5) (end -3.3 0.15) (stroke (width 0.12) (type solid)) (layer "F.SilkS"))
  (fp_line (start -3.3 -2.5) (end 2.55 -2.5) (stroke (width 0.12) (type solid)) (layer "F.SilkS"))
  (fp_line (start -3.3 0.4) (end -3.3 1) (stroke (width 0.12) (type solid)) (layer "F.SilkS"))
  (fp_line (start -3.3 1.25) (end -3.3 4.75) (stroke (width 0.12) (type solid)) (layer "F.SilkS"))
  (fp_line (start -3.3 5) (end -3.3 5.6) (stroke (width 0.12) (type solid)) (layer "F.SilkS"))
  (fp_line (start -3.3 5.9) (end -3.3 8.55) (stroke (width 0.12) (type solid)) (layer "F.SilkS"))
  (fp_line (start -3.3 8.55) (end 2.55 8.55) (stroke (width 0.12) (type solid)) (layer "F.SilkS"))
  (fp_line (start 0 -3) (end 3 -3) (stroke (width 0.12) (type solid)) (layer "F.SilkS"))
  (fp_line (start 2.55 -2.5) (end 2.55 8.55) (stroke (width 0.12) (type solid)) (layer "F.SilkS"))
  (fp_line (start 3 -3) (end 3 0) (stroke (width 0.12) (type solid)) (layer "F.SilkS"))
  (pad "1" thru_hole rect (at 0 0) (size 1.524 1.524) (drill 0.762) (layers "*.Cu" "*.Mask") (remove_unused_layers no) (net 6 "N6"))
  (pad "2" thru_hole circle (at 0 2) (size 1.524 1.524) (drill 0.762) (layers "*.Cu" "*.Mask") (remove_unused_layers no) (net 11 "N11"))
  (pad "3" thru_hole circle (at 0 4) (size 1.524 1.524) (drill 0.762) (layers "*.Cu" "*.Mask") (remove_unused_layers no) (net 15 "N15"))
  (pad "4" thru_hole circle (at 0 6) (size 1.524 1.524) (drill 0.762) (layers "*.Cu" "*.Mask") (remove_unused_layers no) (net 16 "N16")))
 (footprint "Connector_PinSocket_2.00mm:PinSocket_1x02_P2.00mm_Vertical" (layer "F.Cu") (at 193 98)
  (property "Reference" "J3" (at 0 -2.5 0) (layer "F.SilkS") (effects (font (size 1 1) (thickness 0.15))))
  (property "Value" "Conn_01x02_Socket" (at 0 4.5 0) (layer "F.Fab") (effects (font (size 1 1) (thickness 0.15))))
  (fp_line (start -1.06 1) (end -1.06 3.06) (stroke (width 0.12) (type solid)) (layer "F.SilkS"))
  (fp_line (start -1.06 1) (end 1.06 1) (stroke (width 0.12) (type solid)) (layer "F.SilkS"))
  (fp_line (start -1.06 3.06) (end 1.06 3.06) (stroke (width 0.12) (type solid)) (layer "F.SilkS"))
  (fp_line (start 0 -1.06) (end 1.06 -1.06) (stroke (width 0.12) (type solid)) (layer "F.SilkS"))
  (fp_line (start 1.06 -1.06) (end 1.06 0) (stroke (width 0.12) (type solid)) (layer "F.SilkS"))
  (fp_line (start 1.06 1) (end 1.06 3.06) (stroke (width 0.12) (type solid)) (layer "F.SilkS"))
  (pad "1" thru_hole rect (at 0 0) (size 1.35 1.35) (drill 0.8) (layers "*.Cu" "*.Mask") (remove_unused_layers no) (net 33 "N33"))
  (pad "2" thru_hole circle (at 0 2) (size 1.35 1.35) (drill 0.8) (layers "*.Cu" "*.Mask") (remove_unused_layers no) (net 2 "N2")))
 (gr_circle (center 188.239092 85.5) (end 191.239092 85.5) (stroke (width 0.2) (type solid)) (fill no) (layer "Edge.Cuts"))
 (gr_circle (center 113.760908 85.5) (end 116.760908 85.5) (stroke (width 0.2) (type solid)) (fill no) (layer "Edge.Cuts"))
 (gr_circle (center 151 152) (end 154 152) (stroke (width 0.2) (type solid)) (fill no) (layer "Edge.Cuts"))
 (gr_circle (center 151 107) (end 206 107) (stroke (width 0.25) (type solid)) (fill no) (layer "Edge.Cuts"))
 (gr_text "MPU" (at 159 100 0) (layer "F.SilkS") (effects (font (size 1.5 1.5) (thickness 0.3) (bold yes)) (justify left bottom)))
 (segment (start 151.301 74.301) (end 147 70) (width 0.2) (layer "F.Cu") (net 6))
 (segment (start 179 70.5) (end 175.199 74.301) (width 0.2) (layer "F.Cu") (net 6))
 (segment (start 175.199 74.301) (end 151.301 74.301) (width 0.2) (layer "F.Cu") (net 6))
 (segment (start 138.865 108.905) (end 146.8325 100.9375) (width 0.2) (layer "B.Cu") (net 6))
 (segment (start 138.865 119.865) (end 137 121.73) (width 0.2) (layer "B.Cu") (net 6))
 (segment (start 147 100.77) (end 146.8325 100.9375) (width 0.2) (layer "B.Cu") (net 6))
 (segment (start 137 121.73) (end 129.68 121.73) (width 0.2) (layer "B.Cu") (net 6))
 (segment (start 129 70) (end 130.063 68.937) (width 0.2) (layer "B.Cu") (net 6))
 (segment (start 130.063 68.937) (end 145.937 68.937) (width 0.2) (layer "B.Cu") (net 6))
 (segment (start 129.68 121.73) (end 127.22 119.27) (width 0.2) (layer "B.Cu") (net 6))
 (segment (start 145.937 68.937) (end 147 70) (width 0.2) (layer "B.Cu") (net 6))
 (segment (start 138.865 119.865) (end 138.865 108.905) (width 0.2) (layer "B.Cu") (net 6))
 (segment (start 147 70) (end 147 100.77) (width 0.2) (layer "B.Cu") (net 6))
 (segment (start 143 100) (end 143 70) (width 0.2) (layer "B.Cu") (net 8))
 (segment (start 132.3 119.27) (end 133.57 118) (width 0.2) (layer "B.Cu") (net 8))
 (segment (start 142.8325 100.9375) (end 142.8325 100.1675) (width 0.2) (layer "B.Cu") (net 8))
 (segment (start 133.57 118) (end 133.57 110.2) (width 0.2) (layer "B.Cu") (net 8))
 (segment (start 133.57 110.2) (end 142.8325 100.9375) (width 0.2) (layer "B.Cu") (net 8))
 (segment (start 142.8325 100.1675) (end 143 100) (width 0.2) (layer "B.Cu") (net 8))
 (segment (start 145 70) (end 147 68) (width 0.2) (layer "F.Cu") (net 3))
 (segment (start 147 68) (end 171 68) (width 0.2) (layer "F.Cu") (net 3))
 (segment (start 136 109.77) (end 136 117.89) (width 0.2) (layers "B.Cu" "B.Mask") (solder_mask_margin 0.02) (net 3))
 (segment (start 144.8325 100.9375) (end 144.8325 70.1675) (width 0.2) (layer "B.Cu") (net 3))
 (segment (start 144.8325 100.9375) (end 136 109.77) (width 0.2) (layers "B.Cu" "B.Mask") (solder_mask_margin 0.02) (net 3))
 (segment (start 144.8325 70.1675) (end 145 70) (width 0.2) (layer "B.Cu") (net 3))
 (segment (start 170.999922 67.95) (end 179.000078 67.95) (width 0.2) (layer "B.Cu") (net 3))
 (segment (start 136 117.89) (end 137.38 119.27) (width 0.2) (layers "B.Cu" "B.Mask") (solder_mask_margin 0.02) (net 3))
 (segment (start 129.76 119.27) (end 129.76 119.24) (width 0.2) (layer "B.Cu") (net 9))
 (segment (start 140.8325 100.9375) (end 140.8325 70.1675) (width 0.2) (layer "B.Cu") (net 9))
 (segment (start 129.76 119.24) (end 131 118) (width 0.2) (layer "B.Cu") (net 9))
 (segment (start 131 110.77) (end 140.8325 100.9375) (width 0.2) (layer "B.Cu") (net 9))
 (segment (start 131 118) (end 131 110.77) (width 0.2) (layer "B.Cu") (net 9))
 (segment (start 140.8325 70.1675) (end 141 70) (width 0.2) (layer "B.Cu") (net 9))
 (segment (start 126.599 87.636) (end 126.599 74.401) (width 0.2) (layer "F.Cu") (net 11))
 (segment (start 112.235 102) (end 126.599 87.636) (width 0.2) (layer "F.Cu") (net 11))
 (segment (start 126.599 74.401) (end 129 72) (width 0.2) (layer "F.Cu") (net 11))
 (segment (start 117.57 102) (end 112.235 102) (width 0.2) (layer "F.Cu") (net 11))
 (segment (start 132.3 116.73) (end 117.57 102) (width 0.2) (layer "F.Cu") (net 11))
 (segment (start 114.771 104.281) (end 127.22 116.73) (width 0.2) (layer "F.Cu") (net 10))
 (segment (start 109.516 104.281) (end 114.771 104.281) (width 0.2) (layer "F.Cu") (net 10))
 (segment (start 107.235 102) (end 109.516 104.281) (width 0.2) (layer "F.Cu") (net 10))
 (segment (start 111 128) (end 153.431996 128) (width 0.2) (layer "F.Cu") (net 12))
 (segment (start 161.725 119.706996) (end 161.725 118.403004) (width 0.2) (layer "F.Cu") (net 12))
 (segment (start 153.431996 128) (end 161.725 119.706996) (width 0.2) (layer "F.Cu") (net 12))
 (segment (start 164.265 117.785) (end 165.32 116.73) (width 0.2) (layer "F.Cu") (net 12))
 (segment (start 162.343004 117.785) (end 164.265 117.785) (width 0.2) (layer "F.Cu") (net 12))
 (segment (start 161.725 118.403004) (end 162.343004 117.785) (width 0.2) (layer "F.Cu") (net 12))
 (segment (start 159.19 100) (end 142.46 116.73) (width 0.2) (layer "F.Cu") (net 2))
 (segment (start 193 100) (end 159.19 100) (width 0.2) (layer "F.Cu") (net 2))
 (segment (start 141.405 119.706996) (end 141.405 117.785) (width 0.2) (layer "F.Cu") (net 2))
 (segment (start 111 125.46) (end 135.651996 125.46) (width 0.2) (layer "F.Cu") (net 2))
 (segment (start 193 126.46) (end 193 100) (width 0.2) (layer "F.Cu") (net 2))
 (segment (start 141.405 117.785) (end 142.46 116.73) (width 0.2) (layer "F.Cu") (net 2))
 (segment (start 135.651996 125.46) (end 141.405 119.706996) (width 0.2) (layer "F.Cu") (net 2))
 (segment (start 193 129) (end 192.54 129) (width 0.2) (layer "F.Cu") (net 1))
 (segment (start 177.59 129) (end 167.86 119.27) (width 0.2) (layer "F.Cu") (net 1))
 (segment (start 192.54 129) (end 192.49 128.95) (width 0.2) (layer "F.Cu") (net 1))
 (segment (start 193 129) (end 177.59 129) (width 0.2) (layer "F.Cu") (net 1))
 (segment (start 192.95 128.95) (end 193 129) (width 0.2) (layer "B.Cu") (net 1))
 (segment (start 170.999922 70.5) (end 172.300922 71.801) (width 0.2) (layer "B.Cu") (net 4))
 (segment (start 171.860452 117.809548) (end 170.4 119.27) (width 0.2) (layer "B.Cu") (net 4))
 (segment (start 171.860452 115.887552) (end 171.860452 117.809548) (width 0.2) (layer "B.Cu") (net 4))
 (segment (start 172.300922 71.801) (end 172.300922 115.447082) (width 0.2) (layer "B.Cu") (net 4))
 (segment (start 172.300922 115.447082) (end 171.860452 115.887552) (width 0.2) (layer "B.Cu") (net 4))
 (segment (start 170.999922 73) (end 170.999922 85.650078) (width 0.2) (layer "B.Cu") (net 5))
 (segment (start 170.999922 85.650078) (end 139.92 116.73) (width 0.2) (layer "B.Cu") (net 5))
 (segment (start 179 73) (end 172.94 79.06) (width 0.2) (layer "B.Cu") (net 7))
 (segment (start 172.94 79.06) (end 172.94 116.73) (width 0.2) (layer "B.Cu") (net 7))
 (segment (start 171.455 119.706996) (end 171.455 118.833004) (width 0.2) (layer "B.Cu") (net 33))
 (segment (start 172.503004 117.785) (end 176.215 117.785) (width 0.2) (layer "B.Cu") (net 33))
 (segment (start 162.78 119.27) (end 163.835 120.325) (width 0.2) (layer "B.Cu") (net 33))
 (segment (start 176.215 117.785) (end 192.024 101.976) (width 0.2) (layer "B.Cu") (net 33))
 (segment (start 192.024 101.976) (end 192.024 98.976) (width 0.2) (layer "B.Cu") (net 33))
 (segment (start 192.718004 98) (end 193 98) (width 0.2) (layer "B.Cu") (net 33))
 (segment (start 163.835 120.325) (end 170.836996 120.325) (width 0.2) (layer "B.Cu") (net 33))
 (segment (start 170.836996 120.325) (end 171.455 119.706996) (width 0.2) (layer "B.Cu") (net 33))
 (segment (start 171.455 118.833004) (end 172.503004 117.785) (width 0.2) (layer "B.Cu") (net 33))
 (segment (start 192.024 98.976) (end 193 98) (width 0.2) (layer "B.Cu") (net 33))
 (segment (start 137.38 116.73) (end 137.38 84.38) (width 0.2) (layer "F.Cu") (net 16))
 (segment (start 137.38 84.38) (end 129 76) (width 0.2) (layer "F.Cu") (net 16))
 (segment (start 127.937 75.063) (end 129 74) (width 0.2) (layer "F.Cu") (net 15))
 (segment (start 134.84 116.73) (end 127.937 109.827) (width 0.2) (layer "F.Cu") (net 15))
 (segment (start 127.937 109.827) (end 127.937 75.063) (width 0.2) (layer "F.Cu") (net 15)))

